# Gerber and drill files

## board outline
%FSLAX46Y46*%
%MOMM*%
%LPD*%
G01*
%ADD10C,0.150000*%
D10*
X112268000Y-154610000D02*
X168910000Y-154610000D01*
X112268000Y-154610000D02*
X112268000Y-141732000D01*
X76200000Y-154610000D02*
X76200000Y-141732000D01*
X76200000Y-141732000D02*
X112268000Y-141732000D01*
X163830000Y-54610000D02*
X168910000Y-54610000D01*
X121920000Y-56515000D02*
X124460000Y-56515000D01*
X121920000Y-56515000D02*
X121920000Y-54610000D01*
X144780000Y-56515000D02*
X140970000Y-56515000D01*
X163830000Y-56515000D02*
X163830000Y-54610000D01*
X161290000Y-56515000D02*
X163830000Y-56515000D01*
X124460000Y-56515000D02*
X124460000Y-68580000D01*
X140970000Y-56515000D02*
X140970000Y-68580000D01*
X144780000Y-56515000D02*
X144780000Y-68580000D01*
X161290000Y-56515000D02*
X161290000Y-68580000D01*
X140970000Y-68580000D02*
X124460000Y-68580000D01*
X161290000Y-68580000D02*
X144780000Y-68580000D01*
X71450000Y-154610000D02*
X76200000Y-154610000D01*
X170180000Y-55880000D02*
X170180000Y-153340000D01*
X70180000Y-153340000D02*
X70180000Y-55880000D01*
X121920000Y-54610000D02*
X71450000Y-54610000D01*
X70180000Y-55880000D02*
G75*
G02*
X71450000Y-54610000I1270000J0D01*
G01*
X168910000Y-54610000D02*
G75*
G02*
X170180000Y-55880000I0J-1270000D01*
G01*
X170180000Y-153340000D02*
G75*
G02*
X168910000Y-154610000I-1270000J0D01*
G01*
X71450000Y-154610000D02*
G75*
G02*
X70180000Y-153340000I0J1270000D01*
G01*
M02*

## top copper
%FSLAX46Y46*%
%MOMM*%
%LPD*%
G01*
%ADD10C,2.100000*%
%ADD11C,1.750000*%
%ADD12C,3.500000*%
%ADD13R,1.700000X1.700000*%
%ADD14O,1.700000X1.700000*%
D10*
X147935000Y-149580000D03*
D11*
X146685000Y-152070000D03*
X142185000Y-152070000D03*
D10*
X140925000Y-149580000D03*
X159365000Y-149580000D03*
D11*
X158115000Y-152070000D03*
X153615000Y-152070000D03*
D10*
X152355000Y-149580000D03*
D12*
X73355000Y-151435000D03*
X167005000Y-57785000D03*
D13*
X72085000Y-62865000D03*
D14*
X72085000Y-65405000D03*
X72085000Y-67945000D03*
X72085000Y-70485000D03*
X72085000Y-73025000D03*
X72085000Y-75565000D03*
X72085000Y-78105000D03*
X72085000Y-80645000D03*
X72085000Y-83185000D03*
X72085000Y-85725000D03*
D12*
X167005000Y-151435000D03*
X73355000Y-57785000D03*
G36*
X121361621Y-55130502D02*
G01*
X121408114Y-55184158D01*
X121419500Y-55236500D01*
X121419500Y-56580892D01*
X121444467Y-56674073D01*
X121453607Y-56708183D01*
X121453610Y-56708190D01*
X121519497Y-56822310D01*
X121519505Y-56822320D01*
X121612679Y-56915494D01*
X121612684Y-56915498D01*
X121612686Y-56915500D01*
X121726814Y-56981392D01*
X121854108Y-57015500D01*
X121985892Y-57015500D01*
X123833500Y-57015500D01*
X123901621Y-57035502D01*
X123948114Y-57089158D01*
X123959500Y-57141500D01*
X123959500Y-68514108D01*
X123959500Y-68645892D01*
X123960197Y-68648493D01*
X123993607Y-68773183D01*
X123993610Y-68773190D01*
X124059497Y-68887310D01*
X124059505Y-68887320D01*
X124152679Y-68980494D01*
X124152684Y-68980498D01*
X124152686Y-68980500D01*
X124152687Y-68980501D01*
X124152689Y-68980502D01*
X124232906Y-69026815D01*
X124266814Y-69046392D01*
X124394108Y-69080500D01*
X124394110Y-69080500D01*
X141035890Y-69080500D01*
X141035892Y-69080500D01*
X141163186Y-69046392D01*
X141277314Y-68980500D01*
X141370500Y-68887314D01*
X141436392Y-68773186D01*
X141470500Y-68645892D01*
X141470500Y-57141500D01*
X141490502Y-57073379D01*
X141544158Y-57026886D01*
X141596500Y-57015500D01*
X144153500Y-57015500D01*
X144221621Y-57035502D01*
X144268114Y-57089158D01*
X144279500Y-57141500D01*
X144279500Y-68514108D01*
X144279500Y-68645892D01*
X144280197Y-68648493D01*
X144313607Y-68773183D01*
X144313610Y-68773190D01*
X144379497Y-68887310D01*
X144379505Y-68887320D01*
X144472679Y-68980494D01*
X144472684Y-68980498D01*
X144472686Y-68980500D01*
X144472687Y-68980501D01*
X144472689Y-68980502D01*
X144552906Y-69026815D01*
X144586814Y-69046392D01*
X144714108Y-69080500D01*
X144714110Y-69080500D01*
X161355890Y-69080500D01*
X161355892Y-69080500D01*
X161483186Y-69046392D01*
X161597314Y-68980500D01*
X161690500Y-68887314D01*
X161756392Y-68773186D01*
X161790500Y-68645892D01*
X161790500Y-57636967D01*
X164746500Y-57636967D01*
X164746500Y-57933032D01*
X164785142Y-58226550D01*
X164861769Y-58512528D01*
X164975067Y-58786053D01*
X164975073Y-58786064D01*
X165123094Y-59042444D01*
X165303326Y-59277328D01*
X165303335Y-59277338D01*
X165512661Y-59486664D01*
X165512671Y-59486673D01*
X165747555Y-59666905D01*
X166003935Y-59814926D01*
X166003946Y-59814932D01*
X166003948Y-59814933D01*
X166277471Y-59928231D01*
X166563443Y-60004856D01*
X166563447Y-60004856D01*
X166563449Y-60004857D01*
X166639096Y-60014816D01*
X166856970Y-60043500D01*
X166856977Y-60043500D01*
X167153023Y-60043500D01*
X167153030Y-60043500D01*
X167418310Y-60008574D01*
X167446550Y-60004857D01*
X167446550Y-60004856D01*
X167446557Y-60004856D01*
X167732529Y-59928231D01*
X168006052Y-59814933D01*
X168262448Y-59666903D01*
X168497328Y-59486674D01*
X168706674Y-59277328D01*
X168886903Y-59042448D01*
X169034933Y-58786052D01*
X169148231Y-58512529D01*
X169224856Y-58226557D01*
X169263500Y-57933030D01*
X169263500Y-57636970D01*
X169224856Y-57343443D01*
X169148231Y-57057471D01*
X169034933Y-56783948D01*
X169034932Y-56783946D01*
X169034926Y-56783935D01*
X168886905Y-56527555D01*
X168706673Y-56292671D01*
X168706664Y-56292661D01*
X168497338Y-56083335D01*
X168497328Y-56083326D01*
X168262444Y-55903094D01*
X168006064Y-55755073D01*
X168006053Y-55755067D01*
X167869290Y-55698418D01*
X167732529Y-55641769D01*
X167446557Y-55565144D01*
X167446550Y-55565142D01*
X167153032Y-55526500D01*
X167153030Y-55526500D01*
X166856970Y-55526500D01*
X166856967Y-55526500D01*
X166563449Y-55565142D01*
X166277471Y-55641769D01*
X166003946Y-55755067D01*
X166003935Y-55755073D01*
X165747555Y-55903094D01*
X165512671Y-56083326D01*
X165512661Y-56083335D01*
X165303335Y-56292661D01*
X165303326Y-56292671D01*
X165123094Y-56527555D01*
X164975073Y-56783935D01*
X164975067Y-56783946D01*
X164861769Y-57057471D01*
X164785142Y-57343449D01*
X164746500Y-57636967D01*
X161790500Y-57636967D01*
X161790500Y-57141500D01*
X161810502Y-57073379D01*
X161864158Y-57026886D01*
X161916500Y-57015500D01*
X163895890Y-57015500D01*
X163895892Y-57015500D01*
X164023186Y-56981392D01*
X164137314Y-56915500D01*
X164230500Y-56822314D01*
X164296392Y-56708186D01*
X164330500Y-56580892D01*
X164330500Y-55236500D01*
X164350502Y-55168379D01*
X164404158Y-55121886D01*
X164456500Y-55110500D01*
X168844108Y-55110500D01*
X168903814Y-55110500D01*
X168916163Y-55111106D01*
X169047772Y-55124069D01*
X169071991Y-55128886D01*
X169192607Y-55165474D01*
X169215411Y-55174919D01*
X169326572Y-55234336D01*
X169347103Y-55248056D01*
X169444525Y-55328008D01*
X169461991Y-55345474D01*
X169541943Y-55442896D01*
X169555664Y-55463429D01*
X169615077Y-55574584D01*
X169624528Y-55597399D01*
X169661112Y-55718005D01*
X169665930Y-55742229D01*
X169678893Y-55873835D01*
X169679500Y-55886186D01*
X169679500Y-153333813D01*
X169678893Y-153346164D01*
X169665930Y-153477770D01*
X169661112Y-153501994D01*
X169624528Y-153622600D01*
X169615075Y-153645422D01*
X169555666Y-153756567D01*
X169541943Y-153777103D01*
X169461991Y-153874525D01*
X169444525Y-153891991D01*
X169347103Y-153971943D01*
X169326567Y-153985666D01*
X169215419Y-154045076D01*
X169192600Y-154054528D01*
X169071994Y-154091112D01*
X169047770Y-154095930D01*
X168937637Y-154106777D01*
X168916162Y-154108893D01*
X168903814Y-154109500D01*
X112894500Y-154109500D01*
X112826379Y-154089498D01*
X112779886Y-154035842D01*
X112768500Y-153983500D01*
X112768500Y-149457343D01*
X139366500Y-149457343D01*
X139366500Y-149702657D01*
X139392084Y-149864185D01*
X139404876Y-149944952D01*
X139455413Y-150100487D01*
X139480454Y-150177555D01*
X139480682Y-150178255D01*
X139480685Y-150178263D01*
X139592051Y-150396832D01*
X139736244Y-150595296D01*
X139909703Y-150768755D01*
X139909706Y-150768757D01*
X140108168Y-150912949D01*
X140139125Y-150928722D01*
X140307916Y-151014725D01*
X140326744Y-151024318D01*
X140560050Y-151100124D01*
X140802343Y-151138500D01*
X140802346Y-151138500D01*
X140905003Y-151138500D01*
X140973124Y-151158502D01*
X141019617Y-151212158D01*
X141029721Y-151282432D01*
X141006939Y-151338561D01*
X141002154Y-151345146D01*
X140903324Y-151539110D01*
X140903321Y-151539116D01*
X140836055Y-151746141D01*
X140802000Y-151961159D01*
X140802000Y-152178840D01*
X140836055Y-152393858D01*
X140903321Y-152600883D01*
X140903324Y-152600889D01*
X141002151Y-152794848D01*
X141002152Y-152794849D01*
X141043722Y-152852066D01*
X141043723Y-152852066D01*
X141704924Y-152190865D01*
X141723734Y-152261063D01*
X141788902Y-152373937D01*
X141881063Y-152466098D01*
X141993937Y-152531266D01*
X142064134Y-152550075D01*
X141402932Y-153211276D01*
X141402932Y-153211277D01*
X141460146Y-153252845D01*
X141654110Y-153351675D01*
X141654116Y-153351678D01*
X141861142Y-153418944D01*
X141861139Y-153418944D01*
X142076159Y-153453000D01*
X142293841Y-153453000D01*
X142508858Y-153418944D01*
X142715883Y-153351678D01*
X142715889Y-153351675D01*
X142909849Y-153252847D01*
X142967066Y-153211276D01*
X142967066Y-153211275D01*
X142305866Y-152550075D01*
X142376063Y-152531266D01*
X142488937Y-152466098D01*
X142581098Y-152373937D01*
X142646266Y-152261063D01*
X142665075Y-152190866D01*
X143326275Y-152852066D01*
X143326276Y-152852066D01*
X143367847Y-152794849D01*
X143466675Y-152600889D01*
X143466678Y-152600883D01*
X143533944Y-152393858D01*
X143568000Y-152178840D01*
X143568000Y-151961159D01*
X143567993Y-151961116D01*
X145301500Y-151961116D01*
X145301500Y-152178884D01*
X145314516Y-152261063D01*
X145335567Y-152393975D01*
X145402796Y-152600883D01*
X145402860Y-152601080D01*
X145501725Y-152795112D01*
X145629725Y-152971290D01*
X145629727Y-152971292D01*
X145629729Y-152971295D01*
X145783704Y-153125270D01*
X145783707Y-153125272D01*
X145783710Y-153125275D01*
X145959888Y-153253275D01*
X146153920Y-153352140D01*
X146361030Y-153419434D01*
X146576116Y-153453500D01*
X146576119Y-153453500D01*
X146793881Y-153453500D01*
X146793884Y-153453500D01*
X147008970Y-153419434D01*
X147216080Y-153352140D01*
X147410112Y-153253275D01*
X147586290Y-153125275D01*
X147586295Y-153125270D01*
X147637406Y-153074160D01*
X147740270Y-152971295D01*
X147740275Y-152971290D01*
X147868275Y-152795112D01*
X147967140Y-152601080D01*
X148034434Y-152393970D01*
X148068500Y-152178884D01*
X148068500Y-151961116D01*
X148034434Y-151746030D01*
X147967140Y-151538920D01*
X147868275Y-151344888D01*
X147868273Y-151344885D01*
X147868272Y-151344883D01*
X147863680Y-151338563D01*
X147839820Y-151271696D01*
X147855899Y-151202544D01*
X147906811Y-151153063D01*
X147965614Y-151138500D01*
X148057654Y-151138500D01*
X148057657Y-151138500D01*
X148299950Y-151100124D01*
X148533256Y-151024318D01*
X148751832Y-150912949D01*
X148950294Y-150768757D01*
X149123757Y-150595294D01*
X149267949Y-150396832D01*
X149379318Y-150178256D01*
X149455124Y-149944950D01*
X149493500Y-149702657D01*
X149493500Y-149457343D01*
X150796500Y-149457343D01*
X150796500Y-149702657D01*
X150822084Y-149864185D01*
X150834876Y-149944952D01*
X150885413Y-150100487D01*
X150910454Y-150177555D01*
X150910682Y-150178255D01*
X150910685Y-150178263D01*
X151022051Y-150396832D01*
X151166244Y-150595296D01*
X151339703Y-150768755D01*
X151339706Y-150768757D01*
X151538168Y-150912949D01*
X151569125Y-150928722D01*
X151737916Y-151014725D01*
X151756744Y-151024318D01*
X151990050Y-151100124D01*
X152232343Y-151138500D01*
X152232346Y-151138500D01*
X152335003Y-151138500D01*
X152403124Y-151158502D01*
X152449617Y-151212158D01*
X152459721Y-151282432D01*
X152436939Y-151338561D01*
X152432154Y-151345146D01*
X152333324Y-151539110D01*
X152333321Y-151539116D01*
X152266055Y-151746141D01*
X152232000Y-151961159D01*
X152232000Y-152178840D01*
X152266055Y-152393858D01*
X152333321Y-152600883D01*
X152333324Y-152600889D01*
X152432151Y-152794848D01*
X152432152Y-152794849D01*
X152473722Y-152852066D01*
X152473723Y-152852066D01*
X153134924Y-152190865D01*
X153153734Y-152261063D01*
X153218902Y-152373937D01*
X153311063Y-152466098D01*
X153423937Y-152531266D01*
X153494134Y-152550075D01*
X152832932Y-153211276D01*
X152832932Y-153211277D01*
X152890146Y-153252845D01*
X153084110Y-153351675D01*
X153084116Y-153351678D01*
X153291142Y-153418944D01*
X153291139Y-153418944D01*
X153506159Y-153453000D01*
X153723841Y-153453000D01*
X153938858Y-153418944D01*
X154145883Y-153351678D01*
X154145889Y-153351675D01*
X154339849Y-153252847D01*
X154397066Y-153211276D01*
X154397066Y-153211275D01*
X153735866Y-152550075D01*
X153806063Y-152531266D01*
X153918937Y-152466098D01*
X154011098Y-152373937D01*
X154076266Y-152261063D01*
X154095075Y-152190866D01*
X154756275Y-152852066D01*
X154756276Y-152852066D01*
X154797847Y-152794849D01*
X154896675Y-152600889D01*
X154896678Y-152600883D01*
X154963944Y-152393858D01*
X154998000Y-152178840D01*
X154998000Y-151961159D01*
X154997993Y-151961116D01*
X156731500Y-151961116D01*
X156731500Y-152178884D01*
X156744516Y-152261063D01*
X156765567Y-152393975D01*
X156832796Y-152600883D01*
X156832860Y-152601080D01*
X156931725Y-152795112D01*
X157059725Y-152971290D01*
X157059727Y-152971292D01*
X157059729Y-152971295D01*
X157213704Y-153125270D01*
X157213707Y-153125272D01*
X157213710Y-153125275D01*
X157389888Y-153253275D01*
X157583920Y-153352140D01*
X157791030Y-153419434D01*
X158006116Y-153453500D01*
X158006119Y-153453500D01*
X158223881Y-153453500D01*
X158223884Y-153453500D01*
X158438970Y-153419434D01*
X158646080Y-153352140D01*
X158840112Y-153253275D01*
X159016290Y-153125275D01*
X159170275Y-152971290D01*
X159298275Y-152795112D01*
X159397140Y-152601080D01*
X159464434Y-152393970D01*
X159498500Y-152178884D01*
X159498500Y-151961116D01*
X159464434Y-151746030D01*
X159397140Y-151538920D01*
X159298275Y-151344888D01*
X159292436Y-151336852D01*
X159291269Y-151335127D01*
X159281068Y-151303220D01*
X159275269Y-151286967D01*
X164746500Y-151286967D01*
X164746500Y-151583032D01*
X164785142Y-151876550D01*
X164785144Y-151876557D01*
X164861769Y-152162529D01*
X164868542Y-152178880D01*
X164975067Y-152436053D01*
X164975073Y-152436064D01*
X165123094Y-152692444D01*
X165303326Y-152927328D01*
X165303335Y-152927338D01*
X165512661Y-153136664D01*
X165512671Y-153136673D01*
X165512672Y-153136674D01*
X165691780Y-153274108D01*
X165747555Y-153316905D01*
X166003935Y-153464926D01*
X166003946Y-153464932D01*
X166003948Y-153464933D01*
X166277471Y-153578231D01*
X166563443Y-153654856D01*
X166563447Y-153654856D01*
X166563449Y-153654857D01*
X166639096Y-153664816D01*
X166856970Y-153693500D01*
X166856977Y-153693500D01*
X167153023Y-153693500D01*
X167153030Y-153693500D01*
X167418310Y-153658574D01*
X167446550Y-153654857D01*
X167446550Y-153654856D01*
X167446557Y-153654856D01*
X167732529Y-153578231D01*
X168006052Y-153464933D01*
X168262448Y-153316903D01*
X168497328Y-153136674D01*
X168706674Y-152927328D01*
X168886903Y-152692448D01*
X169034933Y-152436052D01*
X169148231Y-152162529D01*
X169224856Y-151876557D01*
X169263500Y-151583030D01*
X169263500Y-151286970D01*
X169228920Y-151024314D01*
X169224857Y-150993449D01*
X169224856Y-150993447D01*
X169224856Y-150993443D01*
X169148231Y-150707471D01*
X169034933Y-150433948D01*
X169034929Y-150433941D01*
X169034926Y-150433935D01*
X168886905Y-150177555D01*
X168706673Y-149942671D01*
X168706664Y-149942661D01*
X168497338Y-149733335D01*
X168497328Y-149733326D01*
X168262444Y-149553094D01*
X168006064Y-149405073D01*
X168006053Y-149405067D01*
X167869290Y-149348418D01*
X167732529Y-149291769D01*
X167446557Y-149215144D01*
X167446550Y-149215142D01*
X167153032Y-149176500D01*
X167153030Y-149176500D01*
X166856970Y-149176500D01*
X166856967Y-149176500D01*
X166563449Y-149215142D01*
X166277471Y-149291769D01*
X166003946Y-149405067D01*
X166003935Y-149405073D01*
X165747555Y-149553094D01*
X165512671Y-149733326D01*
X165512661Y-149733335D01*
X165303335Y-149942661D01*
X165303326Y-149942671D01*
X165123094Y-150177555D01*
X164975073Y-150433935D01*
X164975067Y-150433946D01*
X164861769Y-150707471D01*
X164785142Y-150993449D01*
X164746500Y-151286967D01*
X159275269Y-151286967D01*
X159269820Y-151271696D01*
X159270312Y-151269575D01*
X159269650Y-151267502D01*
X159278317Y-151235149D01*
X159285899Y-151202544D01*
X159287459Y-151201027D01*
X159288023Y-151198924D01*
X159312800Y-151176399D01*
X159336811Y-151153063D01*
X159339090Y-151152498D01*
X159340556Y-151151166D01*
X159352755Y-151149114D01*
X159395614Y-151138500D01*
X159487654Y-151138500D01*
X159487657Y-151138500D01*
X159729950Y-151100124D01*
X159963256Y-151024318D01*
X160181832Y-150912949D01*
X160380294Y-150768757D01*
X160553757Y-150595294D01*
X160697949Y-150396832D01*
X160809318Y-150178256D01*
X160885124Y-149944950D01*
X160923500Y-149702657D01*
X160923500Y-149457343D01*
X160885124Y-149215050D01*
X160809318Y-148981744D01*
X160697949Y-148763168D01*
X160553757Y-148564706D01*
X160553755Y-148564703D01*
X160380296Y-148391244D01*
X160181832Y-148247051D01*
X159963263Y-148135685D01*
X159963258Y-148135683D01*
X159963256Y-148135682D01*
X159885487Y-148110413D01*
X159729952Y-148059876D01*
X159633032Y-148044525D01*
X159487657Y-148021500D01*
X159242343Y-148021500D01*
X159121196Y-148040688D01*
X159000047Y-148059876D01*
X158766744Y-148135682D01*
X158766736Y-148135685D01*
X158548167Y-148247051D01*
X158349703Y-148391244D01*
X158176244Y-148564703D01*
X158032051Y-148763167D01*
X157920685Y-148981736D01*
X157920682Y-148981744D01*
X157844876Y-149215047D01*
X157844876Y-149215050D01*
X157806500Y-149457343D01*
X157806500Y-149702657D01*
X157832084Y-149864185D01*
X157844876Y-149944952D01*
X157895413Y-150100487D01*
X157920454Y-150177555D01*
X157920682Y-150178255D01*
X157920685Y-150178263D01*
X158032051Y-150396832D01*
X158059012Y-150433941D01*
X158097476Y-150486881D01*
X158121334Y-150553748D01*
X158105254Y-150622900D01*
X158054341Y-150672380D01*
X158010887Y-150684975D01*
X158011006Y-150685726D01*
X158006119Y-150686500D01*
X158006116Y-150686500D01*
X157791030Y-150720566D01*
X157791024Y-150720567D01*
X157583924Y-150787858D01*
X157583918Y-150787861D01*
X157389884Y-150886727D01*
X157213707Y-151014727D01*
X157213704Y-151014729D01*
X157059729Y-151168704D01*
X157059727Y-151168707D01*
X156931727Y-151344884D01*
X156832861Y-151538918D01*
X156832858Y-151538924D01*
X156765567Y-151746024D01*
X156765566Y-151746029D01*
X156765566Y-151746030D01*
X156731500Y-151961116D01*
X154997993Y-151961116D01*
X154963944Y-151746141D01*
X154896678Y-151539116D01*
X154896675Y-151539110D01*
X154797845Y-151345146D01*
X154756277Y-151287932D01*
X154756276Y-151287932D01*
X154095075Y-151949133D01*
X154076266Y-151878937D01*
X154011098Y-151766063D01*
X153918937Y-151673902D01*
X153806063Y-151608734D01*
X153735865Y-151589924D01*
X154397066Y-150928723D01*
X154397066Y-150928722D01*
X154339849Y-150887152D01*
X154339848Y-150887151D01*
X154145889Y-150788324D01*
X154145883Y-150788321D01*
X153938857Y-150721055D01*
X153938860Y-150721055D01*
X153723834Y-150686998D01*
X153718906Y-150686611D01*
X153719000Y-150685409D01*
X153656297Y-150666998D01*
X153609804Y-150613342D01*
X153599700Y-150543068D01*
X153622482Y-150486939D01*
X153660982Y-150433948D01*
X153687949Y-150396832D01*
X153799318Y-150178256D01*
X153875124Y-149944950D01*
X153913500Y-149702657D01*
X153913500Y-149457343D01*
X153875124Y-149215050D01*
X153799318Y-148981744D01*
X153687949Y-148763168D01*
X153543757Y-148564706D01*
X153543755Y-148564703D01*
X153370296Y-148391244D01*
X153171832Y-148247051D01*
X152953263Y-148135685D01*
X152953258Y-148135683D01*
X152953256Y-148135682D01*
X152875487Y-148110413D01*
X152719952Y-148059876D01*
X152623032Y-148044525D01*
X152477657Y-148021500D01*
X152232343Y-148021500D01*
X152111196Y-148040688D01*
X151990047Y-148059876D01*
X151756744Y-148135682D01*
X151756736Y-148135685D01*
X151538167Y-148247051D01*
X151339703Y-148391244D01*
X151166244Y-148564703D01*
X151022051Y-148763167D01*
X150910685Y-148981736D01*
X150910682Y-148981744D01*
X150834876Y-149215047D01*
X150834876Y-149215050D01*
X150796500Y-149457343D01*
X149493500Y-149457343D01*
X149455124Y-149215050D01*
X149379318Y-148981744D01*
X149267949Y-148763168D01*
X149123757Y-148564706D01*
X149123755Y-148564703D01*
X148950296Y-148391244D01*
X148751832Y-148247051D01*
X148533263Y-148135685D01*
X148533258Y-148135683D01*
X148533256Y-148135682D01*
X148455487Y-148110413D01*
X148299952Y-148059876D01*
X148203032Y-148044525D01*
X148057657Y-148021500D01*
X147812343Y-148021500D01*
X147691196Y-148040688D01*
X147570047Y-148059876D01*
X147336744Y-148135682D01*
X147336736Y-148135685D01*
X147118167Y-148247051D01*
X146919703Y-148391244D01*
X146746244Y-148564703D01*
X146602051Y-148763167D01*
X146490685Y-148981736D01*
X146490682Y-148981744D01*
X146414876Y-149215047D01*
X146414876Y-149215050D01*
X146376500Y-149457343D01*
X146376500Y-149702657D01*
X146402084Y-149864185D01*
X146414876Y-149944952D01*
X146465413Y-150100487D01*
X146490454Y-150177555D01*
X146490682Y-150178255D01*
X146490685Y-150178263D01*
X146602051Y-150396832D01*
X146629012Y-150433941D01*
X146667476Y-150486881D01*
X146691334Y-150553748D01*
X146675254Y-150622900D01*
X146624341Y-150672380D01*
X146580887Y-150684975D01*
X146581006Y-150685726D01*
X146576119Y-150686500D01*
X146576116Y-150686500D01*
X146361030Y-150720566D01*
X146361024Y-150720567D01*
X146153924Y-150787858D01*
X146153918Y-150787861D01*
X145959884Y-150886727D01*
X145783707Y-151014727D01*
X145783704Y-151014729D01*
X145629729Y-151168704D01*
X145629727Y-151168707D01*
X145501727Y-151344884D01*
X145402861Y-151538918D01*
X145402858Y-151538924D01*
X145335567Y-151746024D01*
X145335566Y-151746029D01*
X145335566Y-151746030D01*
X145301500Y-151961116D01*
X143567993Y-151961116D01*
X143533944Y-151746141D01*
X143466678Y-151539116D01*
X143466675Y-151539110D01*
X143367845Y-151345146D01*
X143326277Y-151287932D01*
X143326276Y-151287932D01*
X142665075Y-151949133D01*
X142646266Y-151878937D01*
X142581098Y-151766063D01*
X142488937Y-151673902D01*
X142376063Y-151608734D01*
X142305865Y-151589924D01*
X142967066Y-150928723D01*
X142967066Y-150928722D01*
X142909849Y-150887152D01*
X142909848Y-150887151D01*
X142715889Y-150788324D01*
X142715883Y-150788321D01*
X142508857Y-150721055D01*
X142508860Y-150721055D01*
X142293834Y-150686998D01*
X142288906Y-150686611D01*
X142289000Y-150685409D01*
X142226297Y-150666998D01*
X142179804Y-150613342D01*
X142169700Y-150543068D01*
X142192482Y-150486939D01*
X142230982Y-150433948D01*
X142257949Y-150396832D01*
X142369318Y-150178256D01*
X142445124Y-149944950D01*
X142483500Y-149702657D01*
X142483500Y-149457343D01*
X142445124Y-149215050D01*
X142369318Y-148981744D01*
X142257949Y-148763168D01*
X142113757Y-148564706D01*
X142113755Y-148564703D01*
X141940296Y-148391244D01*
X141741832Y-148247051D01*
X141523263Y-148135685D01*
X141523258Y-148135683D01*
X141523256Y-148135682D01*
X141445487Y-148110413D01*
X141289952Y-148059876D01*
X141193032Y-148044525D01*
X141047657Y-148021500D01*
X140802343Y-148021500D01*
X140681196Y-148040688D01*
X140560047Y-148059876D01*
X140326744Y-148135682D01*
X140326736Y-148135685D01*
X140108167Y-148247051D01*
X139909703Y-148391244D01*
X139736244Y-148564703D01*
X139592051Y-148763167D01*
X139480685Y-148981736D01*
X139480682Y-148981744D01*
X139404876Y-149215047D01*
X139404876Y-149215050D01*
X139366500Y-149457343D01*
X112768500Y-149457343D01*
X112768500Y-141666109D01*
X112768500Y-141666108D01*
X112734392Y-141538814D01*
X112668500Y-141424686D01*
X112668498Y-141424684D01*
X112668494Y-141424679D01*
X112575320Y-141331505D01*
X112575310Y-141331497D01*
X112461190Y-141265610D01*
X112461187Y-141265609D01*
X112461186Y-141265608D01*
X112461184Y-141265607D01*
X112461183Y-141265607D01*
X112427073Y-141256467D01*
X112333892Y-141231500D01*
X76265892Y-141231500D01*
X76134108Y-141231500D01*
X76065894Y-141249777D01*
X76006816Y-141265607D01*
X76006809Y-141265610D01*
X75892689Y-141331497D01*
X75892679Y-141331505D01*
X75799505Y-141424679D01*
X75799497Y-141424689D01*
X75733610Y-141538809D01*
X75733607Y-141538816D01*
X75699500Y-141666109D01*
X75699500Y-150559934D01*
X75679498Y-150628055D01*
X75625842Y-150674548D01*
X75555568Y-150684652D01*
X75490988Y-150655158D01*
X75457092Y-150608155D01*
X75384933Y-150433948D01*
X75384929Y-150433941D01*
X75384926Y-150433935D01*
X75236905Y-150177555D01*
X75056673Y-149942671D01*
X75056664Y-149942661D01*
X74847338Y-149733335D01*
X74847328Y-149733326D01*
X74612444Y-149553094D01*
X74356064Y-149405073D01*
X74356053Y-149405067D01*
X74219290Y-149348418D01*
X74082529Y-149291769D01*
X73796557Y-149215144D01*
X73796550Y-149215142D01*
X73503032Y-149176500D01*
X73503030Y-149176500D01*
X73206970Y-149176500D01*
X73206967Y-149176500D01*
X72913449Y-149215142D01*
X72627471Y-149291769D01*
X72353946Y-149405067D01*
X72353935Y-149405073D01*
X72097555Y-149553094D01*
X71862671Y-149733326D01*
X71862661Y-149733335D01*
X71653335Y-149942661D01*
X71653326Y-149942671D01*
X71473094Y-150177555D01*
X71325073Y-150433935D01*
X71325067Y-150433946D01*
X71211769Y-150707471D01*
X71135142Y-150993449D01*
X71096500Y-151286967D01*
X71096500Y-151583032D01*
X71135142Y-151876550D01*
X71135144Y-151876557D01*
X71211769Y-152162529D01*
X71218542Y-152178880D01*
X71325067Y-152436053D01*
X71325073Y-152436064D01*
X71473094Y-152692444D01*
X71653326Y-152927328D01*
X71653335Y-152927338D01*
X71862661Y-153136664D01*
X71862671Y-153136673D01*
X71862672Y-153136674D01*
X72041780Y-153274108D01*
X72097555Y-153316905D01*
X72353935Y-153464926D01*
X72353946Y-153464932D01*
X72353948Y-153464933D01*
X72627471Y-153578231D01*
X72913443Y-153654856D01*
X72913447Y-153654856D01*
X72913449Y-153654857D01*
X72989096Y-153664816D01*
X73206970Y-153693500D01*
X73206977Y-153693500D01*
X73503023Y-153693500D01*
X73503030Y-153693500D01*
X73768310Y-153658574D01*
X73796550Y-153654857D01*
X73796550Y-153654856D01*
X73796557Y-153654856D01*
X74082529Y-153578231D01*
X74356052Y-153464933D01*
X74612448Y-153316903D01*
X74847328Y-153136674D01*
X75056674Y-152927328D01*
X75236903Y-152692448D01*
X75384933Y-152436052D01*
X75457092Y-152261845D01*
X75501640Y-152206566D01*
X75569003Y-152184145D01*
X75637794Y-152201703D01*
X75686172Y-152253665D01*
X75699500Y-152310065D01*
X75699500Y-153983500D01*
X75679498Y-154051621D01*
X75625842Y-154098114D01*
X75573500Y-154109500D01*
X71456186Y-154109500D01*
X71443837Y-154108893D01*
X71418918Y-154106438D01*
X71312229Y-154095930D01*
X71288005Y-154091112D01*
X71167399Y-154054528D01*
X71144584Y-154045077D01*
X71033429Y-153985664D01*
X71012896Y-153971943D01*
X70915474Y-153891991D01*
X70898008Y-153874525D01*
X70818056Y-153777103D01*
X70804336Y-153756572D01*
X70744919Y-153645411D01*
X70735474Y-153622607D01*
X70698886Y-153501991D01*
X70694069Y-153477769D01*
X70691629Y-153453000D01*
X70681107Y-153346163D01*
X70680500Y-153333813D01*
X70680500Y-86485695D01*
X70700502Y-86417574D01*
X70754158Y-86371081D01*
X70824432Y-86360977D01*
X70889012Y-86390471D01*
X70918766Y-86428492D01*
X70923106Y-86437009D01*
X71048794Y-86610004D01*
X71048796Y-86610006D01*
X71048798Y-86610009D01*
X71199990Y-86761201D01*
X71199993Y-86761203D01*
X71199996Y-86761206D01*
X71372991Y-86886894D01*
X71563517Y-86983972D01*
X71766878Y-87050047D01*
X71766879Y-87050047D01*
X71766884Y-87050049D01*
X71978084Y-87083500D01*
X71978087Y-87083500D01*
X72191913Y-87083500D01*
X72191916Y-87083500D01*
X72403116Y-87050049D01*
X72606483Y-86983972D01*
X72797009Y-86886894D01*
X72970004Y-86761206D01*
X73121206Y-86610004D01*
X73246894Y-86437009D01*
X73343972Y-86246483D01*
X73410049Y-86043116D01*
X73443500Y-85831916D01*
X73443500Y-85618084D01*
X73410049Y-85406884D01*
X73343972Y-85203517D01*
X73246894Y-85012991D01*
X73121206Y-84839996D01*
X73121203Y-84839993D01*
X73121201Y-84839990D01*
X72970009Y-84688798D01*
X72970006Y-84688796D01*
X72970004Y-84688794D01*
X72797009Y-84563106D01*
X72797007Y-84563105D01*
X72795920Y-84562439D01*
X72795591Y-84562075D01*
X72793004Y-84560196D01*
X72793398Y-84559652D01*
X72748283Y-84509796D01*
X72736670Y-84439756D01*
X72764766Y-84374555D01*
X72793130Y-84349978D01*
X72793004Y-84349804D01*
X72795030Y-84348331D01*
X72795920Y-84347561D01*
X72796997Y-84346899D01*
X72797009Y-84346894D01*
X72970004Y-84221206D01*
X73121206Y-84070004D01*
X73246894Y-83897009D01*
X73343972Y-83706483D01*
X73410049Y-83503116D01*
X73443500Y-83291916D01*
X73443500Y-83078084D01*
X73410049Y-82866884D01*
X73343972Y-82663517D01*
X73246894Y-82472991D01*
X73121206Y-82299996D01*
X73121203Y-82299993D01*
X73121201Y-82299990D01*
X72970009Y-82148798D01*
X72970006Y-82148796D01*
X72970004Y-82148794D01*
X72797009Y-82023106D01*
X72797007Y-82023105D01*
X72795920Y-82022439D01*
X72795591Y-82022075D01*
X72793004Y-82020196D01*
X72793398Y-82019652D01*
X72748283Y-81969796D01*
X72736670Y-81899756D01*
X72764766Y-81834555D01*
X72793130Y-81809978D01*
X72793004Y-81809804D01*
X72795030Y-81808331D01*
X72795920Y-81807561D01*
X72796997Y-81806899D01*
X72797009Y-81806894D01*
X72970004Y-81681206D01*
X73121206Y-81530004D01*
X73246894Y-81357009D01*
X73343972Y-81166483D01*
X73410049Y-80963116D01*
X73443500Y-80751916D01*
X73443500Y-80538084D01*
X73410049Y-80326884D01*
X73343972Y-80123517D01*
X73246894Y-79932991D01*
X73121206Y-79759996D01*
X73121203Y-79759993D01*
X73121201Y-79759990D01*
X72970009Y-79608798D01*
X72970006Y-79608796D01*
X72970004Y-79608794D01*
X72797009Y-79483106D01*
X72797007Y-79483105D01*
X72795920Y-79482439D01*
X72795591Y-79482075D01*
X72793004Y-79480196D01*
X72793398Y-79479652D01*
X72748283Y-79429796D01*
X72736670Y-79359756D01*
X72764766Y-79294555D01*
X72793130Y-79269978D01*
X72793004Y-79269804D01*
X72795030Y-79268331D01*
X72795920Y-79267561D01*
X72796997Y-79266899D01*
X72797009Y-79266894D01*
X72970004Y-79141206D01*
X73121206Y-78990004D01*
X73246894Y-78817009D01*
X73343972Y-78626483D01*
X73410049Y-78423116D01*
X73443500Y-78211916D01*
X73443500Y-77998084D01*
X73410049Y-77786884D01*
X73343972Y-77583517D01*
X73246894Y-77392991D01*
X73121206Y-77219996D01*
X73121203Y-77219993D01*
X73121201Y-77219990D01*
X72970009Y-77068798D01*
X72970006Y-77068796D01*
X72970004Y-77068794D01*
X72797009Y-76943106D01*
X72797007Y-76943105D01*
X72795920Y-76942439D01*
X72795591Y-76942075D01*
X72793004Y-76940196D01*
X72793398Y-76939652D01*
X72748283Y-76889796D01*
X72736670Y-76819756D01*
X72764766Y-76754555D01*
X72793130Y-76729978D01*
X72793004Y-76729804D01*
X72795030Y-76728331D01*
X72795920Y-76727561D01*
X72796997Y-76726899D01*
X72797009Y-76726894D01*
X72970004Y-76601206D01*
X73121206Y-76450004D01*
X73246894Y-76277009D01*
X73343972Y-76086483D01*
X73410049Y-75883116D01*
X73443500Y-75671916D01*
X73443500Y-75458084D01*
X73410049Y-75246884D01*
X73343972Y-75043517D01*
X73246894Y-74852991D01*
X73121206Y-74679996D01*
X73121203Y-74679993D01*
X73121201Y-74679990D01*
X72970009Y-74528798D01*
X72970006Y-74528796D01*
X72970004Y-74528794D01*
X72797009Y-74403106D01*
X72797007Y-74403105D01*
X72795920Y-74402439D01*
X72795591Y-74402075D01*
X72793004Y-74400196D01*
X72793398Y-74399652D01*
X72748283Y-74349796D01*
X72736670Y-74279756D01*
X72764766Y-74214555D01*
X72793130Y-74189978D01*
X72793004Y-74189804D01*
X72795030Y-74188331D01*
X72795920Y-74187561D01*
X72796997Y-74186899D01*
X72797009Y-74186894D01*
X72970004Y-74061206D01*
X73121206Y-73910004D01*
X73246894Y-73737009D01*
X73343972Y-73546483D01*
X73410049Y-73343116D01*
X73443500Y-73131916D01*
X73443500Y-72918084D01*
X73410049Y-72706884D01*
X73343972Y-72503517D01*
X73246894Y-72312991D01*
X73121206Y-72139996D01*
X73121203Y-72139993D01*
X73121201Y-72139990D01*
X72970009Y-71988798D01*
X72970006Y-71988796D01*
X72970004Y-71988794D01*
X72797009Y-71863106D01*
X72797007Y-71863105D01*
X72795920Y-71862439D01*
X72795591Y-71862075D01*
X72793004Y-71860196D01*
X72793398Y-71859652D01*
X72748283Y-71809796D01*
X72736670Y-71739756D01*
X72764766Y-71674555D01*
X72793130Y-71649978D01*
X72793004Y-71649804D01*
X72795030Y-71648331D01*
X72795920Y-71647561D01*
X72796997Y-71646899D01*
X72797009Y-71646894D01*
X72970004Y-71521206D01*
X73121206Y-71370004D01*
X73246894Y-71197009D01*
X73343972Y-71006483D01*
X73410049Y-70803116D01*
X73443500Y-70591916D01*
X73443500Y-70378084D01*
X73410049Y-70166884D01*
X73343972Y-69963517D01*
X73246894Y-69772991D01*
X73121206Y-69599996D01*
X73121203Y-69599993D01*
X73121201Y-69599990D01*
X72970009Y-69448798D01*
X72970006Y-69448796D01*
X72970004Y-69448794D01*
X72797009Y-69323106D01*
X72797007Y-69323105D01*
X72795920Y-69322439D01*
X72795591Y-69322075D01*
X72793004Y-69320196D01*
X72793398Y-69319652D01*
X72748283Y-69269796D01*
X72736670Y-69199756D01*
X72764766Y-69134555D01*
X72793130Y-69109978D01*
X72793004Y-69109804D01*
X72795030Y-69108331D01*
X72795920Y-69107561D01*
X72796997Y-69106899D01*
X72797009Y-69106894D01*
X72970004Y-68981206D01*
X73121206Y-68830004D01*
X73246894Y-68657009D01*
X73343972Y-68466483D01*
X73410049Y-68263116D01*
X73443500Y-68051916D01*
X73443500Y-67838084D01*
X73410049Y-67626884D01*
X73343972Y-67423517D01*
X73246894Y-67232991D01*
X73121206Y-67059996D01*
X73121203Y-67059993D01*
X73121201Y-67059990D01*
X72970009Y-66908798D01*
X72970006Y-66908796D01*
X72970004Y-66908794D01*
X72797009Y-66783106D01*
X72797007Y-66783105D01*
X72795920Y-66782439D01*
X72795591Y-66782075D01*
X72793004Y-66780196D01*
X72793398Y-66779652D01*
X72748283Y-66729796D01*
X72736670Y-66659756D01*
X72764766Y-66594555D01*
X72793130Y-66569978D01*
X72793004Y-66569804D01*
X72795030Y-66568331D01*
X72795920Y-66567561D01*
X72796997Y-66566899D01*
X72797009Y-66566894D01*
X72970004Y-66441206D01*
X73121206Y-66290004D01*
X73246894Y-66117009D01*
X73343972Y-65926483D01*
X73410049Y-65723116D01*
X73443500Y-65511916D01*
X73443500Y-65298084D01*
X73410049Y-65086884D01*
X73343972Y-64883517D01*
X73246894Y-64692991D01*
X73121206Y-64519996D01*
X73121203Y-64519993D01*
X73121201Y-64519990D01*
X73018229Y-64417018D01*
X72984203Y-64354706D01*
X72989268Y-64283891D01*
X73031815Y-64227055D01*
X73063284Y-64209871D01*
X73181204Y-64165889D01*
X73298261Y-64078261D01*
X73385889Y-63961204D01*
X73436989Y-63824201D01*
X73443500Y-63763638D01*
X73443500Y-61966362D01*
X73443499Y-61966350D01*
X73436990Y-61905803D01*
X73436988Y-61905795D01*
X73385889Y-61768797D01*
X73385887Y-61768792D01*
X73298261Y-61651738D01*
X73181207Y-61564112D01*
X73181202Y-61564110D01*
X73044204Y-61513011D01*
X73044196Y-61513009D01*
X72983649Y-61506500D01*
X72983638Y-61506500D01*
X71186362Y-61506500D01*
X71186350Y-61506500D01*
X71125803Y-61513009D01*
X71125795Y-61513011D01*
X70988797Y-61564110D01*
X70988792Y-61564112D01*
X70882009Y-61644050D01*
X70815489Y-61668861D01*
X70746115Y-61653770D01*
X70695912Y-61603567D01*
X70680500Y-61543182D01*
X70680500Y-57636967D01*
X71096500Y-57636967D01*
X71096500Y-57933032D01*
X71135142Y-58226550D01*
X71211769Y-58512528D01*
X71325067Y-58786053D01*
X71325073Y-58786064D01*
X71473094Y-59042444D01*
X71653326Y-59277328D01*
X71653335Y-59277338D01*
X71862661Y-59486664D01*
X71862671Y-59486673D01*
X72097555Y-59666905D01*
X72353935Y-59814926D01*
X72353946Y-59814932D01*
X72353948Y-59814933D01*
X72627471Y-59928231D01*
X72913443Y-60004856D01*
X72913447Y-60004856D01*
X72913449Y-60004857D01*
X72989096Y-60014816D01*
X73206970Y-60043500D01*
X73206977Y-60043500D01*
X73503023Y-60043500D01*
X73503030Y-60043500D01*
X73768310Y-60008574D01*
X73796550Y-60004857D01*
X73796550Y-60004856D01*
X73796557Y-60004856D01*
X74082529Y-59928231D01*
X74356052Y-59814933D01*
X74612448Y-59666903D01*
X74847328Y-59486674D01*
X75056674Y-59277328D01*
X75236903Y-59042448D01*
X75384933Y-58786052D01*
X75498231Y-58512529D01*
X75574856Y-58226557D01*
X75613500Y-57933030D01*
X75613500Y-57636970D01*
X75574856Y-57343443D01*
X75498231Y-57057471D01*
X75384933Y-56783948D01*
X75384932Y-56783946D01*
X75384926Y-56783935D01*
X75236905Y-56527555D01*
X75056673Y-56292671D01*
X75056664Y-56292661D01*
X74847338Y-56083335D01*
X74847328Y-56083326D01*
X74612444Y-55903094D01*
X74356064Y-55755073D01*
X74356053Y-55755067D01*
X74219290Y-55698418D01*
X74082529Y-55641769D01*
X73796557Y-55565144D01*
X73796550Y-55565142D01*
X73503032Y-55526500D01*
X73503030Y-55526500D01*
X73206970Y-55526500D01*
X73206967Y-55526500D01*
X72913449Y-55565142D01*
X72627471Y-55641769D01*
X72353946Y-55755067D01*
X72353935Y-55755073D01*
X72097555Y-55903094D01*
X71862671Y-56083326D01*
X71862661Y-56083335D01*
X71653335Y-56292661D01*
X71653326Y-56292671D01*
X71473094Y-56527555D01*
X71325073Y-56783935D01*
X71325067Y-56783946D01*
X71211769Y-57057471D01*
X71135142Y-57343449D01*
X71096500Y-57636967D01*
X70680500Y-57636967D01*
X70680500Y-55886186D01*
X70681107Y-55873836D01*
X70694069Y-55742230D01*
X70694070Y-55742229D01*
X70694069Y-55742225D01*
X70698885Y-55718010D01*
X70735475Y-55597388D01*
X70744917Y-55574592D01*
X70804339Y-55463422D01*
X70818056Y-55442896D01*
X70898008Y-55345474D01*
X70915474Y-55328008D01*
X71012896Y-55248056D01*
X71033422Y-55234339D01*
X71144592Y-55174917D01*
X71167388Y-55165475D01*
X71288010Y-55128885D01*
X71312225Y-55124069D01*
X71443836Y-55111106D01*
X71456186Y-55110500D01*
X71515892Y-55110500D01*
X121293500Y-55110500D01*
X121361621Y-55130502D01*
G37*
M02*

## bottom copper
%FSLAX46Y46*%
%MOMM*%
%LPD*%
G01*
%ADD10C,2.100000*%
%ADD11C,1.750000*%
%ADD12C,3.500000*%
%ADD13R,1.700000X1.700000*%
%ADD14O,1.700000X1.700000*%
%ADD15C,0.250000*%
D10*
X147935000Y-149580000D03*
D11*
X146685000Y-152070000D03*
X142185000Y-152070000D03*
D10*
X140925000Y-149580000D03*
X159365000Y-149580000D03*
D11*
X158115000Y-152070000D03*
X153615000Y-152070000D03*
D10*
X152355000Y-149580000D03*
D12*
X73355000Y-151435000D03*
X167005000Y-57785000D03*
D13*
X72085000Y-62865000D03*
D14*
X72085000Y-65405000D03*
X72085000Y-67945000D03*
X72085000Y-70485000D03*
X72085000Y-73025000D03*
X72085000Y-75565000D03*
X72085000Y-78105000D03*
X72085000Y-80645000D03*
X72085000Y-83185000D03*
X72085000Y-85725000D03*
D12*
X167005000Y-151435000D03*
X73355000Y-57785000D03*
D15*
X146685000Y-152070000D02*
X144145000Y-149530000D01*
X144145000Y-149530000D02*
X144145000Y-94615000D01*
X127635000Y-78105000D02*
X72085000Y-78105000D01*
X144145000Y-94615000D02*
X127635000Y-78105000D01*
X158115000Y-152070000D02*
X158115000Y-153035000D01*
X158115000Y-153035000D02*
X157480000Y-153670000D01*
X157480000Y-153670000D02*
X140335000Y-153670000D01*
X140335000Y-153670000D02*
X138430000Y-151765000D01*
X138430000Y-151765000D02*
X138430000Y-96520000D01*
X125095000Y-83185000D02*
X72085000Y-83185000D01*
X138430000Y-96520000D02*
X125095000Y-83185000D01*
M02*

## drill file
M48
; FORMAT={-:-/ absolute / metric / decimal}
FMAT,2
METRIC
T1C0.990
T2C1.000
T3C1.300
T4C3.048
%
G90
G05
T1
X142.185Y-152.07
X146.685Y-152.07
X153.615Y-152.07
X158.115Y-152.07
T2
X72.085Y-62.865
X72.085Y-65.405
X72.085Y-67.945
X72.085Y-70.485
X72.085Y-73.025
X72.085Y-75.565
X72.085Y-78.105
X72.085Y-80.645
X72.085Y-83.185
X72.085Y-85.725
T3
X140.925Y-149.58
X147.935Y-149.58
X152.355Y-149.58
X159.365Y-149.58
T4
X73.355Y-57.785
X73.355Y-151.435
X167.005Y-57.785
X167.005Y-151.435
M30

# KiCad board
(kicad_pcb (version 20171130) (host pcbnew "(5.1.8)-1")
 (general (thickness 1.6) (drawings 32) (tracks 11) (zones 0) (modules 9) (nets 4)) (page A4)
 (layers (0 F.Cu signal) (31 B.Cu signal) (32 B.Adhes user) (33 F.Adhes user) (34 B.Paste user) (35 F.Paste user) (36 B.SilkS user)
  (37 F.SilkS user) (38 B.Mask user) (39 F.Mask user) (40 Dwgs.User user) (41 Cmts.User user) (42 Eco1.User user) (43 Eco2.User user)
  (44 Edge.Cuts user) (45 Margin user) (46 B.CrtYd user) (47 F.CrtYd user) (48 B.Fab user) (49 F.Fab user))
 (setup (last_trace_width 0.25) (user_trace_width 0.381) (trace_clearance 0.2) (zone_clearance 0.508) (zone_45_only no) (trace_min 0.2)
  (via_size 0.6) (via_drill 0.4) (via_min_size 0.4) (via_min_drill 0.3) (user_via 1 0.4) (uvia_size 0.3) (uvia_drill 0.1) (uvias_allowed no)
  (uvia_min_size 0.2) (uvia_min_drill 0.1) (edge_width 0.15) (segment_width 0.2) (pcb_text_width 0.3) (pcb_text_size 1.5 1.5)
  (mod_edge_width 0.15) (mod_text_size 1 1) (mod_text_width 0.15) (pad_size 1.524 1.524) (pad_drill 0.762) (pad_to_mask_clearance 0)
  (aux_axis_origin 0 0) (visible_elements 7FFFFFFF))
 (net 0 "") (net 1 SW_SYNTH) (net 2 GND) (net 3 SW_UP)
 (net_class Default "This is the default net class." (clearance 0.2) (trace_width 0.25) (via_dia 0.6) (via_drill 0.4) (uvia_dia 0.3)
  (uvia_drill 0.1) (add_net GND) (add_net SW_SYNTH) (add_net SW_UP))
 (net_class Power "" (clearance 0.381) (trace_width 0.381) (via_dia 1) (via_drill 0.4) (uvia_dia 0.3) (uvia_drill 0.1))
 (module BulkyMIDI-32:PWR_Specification (layer F.Cu) (at 83.185 56.515)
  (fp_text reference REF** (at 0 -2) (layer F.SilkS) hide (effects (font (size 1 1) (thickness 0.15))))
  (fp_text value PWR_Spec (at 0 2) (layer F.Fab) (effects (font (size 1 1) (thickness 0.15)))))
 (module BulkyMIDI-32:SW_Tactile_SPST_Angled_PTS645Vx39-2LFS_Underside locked (layer F.Cu) (at 146.685 152.07 180)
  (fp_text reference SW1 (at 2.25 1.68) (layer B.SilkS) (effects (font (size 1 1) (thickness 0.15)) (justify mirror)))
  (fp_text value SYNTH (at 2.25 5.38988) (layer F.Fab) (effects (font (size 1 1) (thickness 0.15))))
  (pad "" thru_hole circle (at -1.25 2.49 180) (size 2.1 2.1) (drill 1.3) (layers *.Cu *.Mask))
  (pad 2 thru_hole circle (at 0 0 180) (size 1.75 1.75) (drill 0.99) (layers *.Cu *.Mask) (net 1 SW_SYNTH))
  (pad 1 thru_hole circle (at 4.5 0 180) (size 1.75 1.75) (drill 0.99) (layers *.Cu *.Mask) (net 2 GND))
  (pad "" thru_hole circle (at 5.76 2.49 180) (size 2.1 2.1) (drill 1.3) (layers *.Cu *.Mask)))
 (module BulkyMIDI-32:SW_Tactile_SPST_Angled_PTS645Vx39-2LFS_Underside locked (layer F.Cu) (at 158.115 152.07 180)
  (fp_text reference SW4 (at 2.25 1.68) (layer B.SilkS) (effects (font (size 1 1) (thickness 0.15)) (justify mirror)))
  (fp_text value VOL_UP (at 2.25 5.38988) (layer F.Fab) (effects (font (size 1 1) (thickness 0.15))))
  (pad "" thru_hole circle (at -1.25 2.49 180) (size 2.1 2.1) (drill 1.3) (layers *.Cu *.Mask))
  (pad 2 thru_hole circle (at 0 0 180) (size 1.75 1.75) (drill 0.99) (layers *.Cu *.Mask) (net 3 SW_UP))
  (pad 1 thru_hole circle (at 4.5 0 180) (size 1.75 1.75) (drill 0.99) (layers *.Cu *.Mask) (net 2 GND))
  (pad "" thru_hole circle (at 5.76 2.49 180) (size 2.1 2.1) (drill 1.3) (layers *.Cu *.Mask)))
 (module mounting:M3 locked (layer F.Cu) (at 73.355 151.435)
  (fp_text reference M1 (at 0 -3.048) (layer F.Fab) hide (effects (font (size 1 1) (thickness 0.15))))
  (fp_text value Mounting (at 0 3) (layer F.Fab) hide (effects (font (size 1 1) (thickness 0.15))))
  (pad "" np_thru_hole circle (at 0 0) (size 3.5 3.5) (drill 3.048) (layers *.Cu *.Mask) (solder_mask_margin 0.8)))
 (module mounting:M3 (layer F.Cu) (at 167.005 57.785)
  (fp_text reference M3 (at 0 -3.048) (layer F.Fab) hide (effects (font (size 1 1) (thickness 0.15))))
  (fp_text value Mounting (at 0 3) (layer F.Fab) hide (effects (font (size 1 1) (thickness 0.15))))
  (pad "" np_thru_hole circle (at 0 0) (size 3.5 3.5) (drill 3.048) (layers *.Cu *.Mask) (solder_mask_margin 0.8)))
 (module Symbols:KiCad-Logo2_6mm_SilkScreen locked (layer B.Cu) (at 99.695 79.375 180)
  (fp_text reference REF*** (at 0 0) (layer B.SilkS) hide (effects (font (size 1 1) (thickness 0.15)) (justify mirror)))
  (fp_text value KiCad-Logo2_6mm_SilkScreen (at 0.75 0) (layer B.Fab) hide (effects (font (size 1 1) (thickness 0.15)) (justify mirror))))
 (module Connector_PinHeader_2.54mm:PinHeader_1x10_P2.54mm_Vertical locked (layer B.Cu) (at 72.085 62.865 180)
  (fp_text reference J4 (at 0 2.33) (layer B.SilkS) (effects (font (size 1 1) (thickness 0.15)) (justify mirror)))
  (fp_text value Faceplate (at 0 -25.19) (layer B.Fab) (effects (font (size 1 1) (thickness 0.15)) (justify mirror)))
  (pad 1 thru_hole rect (at 0 0 180) (size 1.7 1.7) (drill 1) (layers *.Cu *.Mask))
  (pad 2 thru_hole oval (at 0 -2.54 180) (size 1.7 1.7) (drill 1) (layers *.Cu *.Mask))
  (pad 3 thru_hole oval (at 0 -5.08 180) (size 1.7 1.7) (drill 1) (layers *.Cu *.Mask))
  (pad 4 thru_hole oval (at 0 -7.62 180) (size 1.7 1.7) (drill 1) (layers *.Cu *.Mask))
  (pad 5 thru_hole oval (at 0 -10.16 180) (size 1.7 1.7) (drill 1) (layers *.Cu *.Mask))
  (pad 6 thru_hole oval (at 0 -12.7 180) (size 1.7 1.7) (drill 1) (layers *.Cu *.Mask))
  (pad 7 thru_hole oval (at 0 -15.24 180) (size 1.7 1.7) (drill 1) (layers *.Cu *.Mask) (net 1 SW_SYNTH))
  (pad 8 thru_hole oval (at 0 -17.78 180) (size 1.7 1.7) (drill 1) (layers *.Cu *.Mask))
  (pad 9 thru_hole oval (at 0 -20.32 180) (size 1.7 1.7) (drill 1) (layers *.Cu *.Mask) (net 3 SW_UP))
  (pad 10 thru_hole oval (at 0 -22.86 180) (size 1.7 1.7) (drill 1) (layers *.Cu *.Mask)))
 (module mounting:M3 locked (layer F.Cu) (at 167.005 151.435)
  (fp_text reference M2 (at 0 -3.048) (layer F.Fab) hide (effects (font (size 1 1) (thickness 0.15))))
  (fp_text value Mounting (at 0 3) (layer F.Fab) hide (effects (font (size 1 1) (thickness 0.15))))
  (pad "" np_thru_hole circle (at 0 0) (size 3.5 3.5) (drill 3.048) (layers *.Cu *.Mask) (solder_mask_margin 0.8)))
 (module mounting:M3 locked (layer F.Cu) (at 73.355 57.785)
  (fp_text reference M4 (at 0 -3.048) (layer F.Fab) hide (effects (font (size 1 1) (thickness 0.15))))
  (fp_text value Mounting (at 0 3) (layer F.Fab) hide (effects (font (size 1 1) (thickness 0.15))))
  (pad "" np_thru_hole circle (at 0 0) (size 3.5 3.5) (drill 3.048) (layers *.Cu *.Mask) (solder_mask_margin 0.8)))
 (gr_line (start 112.268 154.61) (end 168.91 154.61) (layer Edge.Cuts) (width 0.15))
 (gr_line (start 112.268 154.61) (end 112.268 141.732) (layer Edge.Cuts) (width 0.15))
 (gr_line (start 76.2 154.61) (end 76.2 141.732) (layer Edge.Cuts) (width 0.15))
 (gr_line (start 76.2 141.732) (end 112.268 141.732) (layer Edge.Cuts) (width 0.15))
 (gr_line (start 163.83 54.61) (end 168.91 54.61) (layer Edge.Cuts) (width 0.15))
 (gr_line (start 121.92 56.515) (end 124.46 56.515) (layer Edge.Cuts) (width 0.15))
 (gr_line (start 121.92 56.515) (end 121.92 54.61) (layer Edge.Cuts) (width 0.15))
 (gr_line (start 144.78 56.515) (end 140.97 56.515) (layer Edge.Cuts) (width 0.15))
 (gr_line (start 163.83 56.515) (end 163.83 54.61) (layer Edge.Cuts) (width 0.15))
 (gr_line (start 161.29 56.515) (end 163.83 56.515) (layer Edge.Cuts) (width 0.15))
 (gr_line (start 124.46 56.515) (end 124.46 68.58) (layer Edge.Cuts) (width 0.15))
 (gr_line (start 140.97 56.515) (end 140.97 68.58) (layer Edge.Cuts) (width 0.15))
 (gr_line (start 144.78 56.515) (end 144.78 68.58) (layer Edge.Cuts) (width 0.15))
 (gr_line (start 161.29 56.515) (end 161.29 68.58) (layer Edge.Cuts) (width 0.15))
 (gr_line (start 140.97 68.58) (end 124.46 68.58) (layer Edge.Cuts) (width 0.15))
 (gr_line (start 161.29 68.58) (end 144.78 68.58) (layer Edge.Cuts) (width 0.15))
 (gr_line (start 71.45 154.61) (end 76.2 154.61) (layer Edge.Cuts) (width 0.15))
 (gr_line (start 170.18 55.88) (end 170.18 153.34) (layer Edge.Cuts) (width 0.15))
 (gr_line (start 70.18 153.34) (end 70.18 55.88) (layer Edge.Cuts) (width 0.15))
 (gr_line (start 121.92 54.61) (end 71.45 54.61) (angle 90) (layer Edge.Cuts) (width 0.15))
 (gr_arc (start 71.45 55.88) (end 70.18 55.88) (angle 90) (layer Edge.Cuts) (width 0.15))
 (gr_arc (start 168.91 55.88) (end 168.91 54.61) (angle 90) (layer Edge.Cuts) (width 0.15))
 (gr_arc (start 168.91 153.34) (end 170.18 153.34) (angle 90) (layer Edge.Cuts) (width 0.15))
 (gr_arc (start 71.45 153.34) (end 71.45 154.61) (angle 90) (layer Edge.Cuts) (width 0.15))
 (segment (start 146.685 152.07) (end 144.145 149.53) (width 0.25) (layer B.Cu) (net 1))
 (segment (start 144.145 149.53) (end 144.145 94.615) (width 0.25) (layer B.Cu) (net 1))
 (segment (start 127.635 78.105) (end 72.085 78.105) (width 0.25) (layer B.Cu) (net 1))
 (segment (start 144.145 94.615) (end 127.635 78.105) (width 0.25) (layer B.Cu) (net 1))
 (segment (start 158.115 152.07) (end 158.115 153.035) (width 0.25) (layer B.Cu) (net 3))
 (segment (start 158.115 153.035) (end 157.48 153.67) (width 0.25) (layer B.Cu) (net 3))
 (segment (start 157.48 153.67) (end 140.335 153.67) (width 0.25) (layer B.Cu) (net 3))
 (segment (start 140.335 153.67) (end 138.43 151.765) (width 0.25) (layer B.Cu) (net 3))
 (segment (start 138.43 151.765) (end 138.43 96.52) (width 0.25) (layer B.Cu) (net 3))
 (segment (start 125.095 83.185) (end 72.085 83.185) (width 0.25) (layer B.Cu) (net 3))
 (segment (start 138.43 96.52) (end 125.095 83.185) (width 0.25) (layer B.Cu) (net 3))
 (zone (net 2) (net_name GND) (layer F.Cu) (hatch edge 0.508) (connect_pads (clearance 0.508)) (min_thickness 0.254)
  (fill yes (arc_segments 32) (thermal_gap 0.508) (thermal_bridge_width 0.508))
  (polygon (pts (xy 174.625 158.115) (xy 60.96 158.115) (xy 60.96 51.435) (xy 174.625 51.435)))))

